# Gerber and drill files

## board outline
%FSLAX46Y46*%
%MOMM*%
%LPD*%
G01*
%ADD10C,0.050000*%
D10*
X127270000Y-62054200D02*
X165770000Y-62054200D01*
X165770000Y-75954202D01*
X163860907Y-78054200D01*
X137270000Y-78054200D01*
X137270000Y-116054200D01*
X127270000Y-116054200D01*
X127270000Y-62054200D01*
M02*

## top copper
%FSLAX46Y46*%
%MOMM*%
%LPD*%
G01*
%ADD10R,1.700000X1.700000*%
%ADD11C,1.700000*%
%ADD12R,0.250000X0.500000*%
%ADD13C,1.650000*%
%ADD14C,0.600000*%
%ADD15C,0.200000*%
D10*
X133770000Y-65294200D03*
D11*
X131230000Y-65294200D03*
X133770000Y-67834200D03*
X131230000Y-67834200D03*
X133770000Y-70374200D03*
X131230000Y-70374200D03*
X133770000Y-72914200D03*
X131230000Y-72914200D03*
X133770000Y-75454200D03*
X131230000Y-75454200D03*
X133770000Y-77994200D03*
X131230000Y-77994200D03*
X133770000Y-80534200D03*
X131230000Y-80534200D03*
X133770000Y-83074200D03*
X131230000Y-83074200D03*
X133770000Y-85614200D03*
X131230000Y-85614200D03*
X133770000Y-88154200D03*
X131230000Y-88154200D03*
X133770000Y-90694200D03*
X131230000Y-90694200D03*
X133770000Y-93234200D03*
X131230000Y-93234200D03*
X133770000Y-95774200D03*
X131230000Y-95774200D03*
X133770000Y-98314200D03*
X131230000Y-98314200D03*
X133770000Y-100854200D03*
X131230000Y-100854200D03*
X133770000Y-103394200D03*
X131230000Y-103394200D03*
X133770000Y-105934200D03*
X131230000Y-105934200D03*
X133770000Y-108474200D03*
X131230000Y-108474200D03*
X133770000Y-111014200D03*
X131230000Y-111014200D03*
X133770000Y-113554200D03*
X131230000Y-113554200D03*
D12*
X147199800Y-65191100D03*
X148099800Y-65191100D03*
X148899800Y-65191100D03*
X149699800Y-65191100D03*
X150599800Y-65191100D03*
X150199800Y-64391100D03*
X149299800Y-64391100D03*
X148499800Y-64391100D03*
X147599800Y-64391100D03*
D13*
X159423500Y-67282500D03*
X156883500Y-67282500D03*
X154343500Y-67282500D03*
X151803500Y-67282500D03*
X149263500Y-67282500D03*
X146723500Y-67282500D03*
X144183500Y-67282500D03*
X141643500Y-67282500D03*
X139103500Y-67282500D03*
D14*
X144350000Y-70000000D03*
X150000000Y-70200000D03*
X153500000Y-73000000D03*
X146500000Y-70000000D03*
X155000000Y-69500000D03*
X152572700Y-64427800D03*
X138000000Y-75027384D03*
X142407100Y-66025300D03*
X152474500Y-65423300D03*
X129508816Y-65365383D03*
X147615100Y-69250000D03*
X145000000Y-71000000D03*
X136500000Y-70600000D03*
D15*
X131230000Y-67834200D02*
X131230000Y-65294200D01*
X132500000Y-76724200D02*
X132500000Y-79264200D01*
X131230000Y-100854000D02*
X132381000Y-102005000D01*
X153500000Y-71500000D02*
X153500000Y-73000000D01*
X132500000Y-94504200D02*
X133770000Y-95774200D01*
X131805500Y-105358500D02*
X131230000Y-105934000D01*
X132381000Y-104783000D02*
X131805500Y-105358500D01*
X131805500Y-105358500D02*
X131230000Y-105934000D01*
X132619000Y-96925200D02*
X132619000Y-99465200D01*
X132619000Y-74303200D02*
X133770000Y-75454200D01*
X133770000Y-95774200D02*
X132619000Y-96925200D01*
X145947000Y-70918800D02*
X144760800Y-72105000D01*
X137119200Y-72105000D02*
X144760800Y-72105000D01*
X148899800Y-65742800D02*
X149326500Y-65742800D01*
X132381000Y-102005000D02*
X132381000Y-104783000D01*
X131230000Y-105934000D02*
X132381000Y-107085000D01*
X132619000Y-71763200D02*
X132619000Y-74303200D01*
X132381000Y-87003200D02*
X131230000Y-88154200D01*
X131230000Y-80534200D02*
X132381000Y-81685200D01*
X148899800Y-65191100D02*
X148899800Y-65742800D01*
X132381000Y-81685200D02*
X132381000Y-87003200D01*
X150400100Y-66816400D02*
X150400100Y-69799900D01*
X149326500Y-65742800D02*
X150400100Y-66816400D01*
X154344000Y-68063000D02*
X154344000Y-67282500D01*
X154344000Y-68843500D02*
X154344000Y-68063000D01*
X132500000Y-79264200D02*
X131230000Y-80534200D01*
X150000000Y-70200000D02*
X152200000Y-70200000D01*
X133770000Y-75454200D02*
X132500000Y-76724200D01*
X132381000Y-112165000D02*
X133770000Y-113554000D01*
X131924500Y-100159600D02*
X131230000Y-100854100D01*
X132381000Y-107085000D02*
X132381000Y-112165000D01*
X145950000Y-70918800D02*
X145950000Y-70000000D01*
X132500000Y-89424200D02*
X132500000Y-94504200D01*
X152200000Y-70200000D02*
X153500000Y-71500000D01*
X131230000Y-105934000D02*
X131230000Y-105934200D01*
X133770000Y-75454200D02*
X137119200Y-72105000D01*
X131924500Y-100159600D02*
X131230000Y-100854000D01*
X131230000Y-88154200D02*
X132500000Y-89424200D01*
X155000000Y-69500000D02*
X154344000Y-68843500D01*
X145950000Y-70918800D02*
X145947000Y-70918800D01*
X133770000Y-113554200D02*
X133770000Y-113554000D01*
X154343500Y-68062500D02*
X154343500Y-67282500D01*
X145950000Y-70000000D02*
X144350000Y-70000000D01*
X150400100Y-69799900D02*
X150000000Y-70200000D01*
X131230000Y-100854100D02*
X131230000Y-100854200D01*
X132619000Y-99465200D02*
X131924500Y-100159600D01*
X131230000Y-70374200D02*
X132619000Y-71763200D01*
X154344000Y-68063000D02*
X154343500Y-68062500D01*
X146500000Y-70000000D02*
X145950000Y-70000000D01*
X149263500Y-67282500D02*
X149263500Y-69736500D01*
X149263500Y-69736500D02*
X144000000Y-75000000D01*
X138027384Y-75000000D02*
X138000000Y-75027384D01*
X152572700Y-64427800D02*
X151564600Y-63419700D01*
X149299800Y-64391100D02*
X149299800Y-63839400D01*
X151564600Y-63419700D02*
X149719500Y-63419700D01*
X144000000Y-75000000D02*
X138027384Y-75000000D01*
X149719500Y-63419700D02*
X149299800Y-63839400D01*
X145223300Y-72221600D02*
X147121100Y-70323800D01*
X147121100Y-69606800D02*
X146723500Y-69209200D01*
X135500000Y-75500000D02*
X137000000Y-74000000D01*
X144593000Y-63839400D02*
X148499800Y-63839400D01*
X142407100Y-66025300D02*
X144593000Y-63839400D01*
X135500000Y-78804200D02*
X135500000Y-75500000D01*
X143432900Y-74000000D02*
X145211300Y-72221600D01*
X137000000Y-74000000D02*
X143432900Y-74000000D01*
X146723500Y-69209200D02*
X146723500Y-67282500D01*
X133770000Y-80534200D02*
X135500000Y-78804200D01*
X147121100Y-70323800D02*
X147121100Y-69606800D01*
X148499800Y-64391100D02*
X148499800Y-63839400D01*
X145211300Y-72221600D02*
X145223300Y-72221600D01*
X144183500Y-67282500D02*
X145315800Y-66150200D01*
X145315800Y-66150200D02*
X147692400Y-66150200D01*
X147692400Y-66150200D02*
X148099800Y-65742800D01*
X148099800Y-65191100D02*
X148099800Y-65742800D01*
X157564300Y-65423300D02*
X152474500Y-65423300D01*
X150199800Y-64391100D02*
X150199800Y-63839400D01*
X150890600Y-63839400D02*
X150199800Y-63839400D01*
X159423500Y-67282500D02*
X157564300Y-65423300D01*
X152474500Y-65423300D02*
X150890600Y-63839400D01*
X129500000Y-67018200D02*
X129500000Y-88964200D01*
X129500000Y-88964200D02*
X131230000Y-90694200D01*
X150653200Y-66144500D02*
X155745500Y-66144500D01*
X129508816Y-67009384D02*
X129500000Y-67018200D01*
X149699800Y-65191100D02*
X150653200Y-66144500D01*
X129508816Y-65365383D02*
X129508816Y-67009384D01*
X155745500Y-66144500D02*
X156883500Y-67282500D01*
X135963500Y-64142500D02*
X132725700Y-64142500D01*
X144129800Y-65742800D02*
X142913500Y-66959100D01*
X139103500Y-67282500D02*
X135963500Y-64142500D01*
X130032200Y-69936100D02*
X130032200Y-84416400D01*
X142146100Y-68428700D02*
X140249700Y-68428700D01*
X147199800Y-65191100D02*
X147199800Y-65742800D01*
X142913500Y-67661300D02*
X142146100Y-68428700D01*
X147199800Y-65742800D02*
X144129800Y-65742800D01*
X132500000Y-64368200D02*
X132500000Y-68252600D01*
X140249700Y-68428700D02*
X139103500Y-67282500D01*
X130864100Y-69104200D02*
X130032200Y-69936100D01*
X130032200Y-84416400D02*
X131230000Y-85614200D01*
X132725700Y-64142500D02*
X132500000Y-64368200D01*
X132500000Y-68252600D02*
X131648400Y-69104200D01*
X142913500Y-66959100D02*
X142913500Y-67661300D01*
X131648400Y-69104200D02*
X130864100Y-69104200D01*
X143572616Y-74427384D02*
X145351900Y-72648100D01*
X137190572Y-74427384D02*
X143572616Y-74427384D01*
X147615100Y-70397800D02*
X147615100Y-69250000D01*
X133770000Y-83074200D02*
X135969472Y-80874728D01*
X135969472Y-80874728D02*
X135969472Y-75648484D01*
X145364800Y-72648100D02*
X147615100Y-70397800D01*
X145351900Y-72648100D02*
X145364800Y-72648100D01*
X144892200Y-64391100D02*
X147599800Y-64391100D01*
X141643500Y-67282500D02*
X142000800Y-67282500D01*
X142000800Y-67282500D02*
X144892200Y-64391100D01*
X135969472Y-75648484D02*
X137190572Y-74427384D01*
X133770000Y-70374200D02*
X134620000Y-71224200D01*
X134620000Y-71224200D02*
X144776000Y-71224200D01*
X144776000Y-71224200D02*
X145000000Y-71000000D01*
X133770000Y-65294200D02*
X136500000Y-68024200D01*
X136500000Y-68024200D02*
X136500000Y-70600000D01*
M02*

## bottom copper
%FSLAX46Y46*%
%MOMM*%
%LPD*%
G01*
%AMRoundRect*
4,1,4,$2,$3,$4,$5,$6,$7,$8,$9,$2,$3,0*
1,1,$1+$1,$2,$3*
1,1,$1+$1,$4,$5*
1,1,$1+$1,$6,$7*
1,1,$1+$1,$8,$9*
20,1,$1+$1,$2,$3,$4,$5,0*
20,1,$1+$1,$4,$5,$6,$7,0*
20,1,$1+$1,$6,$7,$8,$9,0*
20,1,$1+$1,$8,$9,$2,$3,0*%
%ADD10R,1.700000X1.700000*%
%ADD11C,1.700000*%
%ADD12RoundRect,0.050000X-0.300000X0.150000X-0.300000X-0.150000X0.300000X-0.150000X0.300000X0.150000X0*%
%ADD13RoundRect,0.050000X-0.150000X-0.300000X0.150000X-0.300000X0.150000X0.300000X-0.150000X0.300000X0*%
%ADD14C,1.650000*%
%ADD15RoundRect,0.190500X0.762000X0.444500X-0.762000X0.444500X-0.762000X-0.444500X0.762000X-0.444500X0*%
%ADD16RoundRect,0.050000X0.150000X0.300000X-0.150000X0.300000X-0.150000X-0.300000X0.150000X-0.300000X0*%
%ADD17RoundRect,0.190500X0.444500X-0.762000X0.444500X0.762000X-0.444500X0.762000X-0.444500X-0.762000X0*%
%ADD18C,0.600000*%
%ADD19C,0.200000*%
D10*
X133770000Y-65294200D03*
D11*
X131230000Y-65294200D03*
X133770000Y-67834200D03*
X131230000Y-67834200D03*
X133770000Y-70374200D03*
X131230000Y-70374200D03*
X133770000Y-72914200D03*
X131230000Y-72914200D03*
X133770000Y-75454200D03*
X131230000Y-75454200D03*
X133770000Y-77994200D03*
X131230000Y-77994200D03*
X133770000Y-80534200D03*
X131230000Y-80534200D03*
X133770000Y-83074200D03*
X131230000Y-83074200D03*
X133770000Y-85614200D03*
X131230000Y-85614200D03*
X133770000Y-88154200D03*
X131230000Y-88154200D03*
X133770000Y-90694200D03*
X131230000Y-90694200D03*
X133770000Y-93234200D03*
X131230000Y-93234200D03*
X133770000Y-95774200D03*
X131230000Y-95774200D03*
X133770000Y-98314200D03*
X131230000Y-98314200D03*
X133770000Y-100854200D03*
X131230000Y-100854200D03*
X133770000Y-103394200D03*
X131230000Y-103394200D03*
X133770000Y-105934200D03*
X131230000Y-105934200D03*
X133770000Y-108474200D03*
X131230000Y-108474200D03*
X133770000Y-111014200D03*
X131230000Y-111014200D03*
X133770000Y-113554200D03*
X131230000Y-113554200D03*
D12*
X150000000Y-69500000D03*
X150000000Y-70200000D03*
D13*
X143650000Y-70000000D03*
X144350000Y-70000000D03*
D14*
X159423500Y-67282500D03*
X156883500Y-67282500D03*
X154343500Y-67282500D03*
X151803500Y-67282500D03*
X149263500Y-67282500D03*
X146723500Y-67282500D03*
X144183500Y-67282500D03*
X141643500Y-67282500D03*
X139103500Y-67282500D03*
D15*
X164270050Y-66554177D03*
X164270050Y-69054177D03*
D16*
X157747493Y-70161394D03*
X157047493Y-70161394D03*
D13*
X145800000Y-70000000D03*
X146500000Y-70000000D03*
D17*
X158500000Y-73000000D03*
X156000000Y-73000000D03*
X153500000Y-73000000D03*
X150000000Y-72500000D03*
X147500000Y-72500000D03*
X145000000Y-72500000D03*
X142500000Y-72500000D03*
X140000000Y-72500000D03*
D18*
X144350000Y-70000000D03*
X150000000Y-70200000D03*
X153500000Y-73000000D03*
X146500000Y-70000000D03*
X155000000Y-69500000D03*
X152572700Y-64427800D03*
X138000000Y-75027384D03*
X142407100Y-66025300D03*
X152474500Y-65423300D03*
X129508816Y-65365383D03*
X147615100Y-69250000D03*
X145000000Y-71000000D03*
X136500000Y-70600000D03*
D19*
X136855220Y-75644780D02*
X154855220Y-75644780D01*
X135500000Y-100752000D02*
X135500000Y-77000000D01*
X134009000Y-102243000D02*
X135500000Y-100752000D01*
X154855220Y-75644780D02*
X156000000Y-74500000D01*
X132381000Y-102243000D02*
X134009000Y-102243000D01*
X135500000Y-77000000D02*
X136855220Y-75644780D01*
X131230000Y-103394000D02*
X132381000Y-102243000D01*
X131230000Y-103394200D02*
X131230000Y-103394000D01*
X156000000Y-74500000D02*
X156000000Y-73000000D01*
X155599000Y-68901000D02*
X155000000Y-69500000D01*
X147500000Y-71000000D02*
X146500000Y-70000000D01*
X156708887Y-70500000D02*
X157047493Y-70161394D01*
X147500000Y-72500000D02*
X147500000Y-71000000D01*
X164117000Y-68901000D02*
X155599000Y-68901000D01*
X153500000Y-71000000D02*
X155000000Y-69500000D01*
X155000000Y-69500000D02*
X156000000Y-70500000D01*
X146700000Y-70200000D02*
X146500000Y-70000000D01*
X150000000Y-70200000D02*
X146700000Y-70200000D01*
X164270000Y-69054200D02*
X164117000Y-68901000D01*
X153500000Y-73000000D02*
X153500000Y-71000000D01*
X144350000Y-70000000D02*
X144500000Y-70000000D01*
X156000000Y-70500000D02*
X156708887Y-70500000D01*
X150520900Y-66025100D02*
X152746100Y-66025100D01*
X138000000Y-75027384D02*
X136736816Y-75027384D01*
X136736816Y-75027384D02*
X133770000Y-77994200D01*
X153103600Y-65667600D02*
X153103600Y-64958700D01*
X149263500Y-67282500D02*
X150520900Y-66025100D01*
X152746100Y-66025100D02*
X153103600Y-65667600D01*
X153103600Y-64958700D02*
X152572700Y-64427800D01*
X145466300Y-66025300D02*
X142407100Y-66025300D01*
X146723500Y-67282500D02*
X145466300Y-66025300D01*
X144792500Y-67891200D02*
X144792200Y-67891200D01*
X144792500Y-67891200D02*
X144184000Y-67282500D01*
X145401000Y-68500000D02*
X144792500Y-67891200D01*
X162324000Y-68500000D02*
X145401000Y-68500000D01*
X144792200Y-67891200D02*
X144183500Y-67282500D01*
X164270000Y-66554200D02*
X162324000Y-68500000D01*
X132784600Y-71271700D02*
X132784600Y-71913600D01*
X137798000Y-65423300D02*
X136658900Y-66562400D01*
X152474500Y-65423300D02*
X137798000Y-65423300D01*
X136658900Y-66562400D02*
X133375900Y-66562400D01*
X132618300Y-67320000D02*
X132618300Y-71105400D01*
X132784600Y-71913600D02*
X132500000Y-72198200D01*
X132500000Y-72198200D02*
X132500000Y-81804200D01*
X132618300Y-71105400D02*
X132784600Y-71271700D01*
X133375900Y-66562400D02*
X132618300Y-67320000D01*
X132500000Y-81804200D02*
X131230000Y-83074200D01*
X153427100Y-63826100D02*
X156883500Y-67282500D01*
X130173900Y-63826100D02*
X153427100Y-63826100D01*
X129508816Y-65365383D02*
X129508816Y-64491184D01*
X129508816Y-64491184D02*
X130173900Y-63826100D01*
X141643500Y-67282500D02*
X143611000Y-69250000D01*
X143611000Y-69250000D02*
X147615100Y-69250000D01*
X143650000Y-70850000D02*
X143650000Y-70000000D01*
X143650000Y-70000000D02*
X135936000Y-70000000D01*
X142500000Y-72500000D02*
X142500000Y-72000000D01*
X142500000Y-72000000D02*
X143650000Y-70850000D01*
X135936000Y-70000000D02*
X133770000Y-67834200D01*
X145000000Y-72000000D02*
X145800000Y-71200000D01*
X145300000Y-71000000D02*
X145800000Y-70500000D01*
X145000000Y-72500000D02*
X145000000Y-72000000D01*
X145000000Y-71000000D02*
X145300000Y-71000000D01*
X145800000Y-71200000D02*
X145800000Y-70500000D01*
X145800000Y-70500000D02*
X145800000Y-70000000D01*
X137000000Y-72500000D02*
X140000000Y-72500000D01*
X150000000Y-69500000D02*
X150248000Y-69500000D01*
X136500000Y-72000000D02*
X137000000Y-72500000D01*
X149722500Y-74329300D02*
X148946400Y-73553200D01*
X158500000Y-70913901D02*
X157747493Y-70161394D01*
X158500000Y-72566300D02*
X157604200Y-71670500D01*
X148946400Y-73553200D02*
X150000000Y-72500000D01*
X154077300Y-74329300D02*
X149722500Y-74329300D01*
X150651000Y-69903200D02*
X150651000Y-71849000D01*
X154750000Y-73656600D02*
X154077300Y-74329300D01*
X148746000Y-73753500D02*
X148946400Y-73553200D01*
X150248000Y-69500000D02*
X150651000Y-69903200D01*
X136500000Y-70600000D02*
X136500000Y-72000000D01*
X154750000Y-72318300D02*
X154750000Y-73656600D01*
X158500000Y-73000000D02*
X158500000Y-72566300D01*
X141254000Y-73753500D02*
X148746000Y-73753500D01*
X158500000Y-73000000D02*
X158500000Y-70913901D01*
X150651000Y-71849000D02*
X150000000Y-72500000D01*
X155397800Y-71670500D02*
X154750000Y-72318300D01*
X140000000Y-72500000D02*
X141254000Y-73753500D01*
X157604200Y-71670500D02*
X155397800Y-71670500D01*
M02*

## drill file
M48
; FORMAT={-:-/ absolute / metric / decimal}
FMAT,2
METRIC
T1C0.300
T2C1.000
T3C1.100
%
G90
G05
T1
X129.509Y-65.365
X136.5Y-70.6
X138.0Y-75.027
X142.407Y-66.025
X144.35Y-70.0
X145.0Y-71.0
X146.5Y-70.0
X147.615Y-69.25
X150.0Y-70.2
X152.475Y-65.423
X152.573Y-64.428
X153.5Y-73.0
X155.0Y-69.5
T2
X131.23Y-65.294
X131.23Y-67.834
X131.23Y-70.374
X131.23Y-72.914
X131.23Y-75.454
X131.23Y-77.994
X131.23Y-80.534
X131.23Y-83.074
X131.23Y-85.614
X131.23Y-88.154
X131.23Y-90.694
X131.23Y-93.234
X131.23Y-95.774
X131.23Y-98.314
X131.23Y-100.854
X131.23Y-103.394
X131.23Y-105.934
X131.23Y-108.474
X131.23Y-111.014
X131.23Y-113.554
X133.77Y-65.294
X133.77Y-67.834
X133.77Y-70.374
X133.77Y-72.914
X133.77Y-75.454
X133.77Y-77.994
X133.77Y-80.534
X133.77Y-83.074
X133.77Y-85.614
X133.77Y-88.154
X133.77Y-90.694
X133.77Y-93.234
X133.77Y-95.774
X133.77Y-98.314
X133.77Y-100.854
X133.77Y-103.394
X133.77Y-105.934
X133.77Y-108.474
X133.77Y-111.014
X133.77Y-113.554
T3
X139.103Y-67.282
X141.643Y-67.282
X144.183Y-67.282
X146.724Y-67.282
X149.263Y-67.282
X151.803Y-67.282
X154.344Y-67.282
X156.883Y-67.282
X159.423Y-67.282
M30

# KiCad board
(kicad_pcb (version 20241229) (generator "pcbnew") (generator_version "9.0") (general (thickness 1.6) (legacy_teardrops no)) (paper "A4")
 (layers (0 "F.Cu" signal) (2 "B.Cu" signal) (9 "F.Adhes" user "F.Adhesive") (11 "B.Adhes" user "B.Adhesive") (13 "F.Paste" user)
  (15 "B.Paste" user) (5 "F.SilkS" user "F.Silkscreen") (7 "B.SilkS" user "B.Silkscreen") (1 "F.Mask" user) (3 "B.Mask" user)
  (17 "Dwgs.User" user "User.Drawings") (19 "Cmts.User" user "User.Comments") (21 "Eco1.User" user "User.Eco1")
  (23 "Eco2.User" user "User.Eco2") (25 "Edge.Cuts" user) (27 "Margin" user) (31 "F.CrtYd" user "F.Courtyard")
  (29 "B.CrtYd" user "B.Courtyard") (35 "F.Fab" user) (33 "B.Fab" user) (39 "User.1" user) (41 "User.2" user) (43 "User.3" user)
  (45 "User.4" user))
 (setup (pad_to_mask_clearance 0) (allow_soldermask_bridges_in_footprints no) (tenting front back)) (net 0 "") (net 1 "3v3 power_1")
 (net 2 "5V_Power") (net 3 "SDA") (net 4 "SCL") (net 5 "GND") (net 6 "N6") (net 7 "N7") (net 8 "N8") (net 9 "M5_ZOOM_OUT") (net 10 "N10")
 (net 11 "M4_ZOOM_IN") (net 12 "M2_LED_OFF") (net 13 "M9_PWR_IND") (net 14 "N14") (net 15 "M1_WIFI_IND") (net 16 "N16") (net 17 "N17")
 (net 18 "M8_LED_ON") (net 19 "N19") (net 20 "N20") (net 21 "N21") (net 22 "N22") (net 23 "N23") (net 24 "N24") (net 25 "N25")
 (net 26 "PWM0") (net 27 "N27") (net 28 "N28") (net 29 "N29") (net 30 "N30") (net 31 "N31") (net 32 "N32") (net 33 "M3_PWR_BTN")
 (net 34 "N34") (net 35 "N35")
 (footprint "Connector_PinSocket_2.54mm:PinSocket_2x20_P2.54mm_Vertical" (layer "F.Cu") (at 133.77 65.2942)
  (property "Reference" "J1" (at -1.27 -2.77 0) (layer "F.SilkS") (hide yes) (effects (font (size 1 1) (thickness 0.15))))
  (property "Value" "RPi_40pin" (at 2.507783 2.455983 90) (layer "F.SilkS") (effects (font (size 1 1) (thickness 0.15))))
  (pad "1" thru_hole rect (at 0 0) (size 1.7 1.7) (drill 1) (layers "*.Cu" "*.Mask") (remove_unused_layers no) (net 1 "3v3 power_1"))
  (pad "2" thru_hole circle (at -2.54 0) (size 1.7 1.7) (drill 1) (layers "*.Cu" "*.Mask") (remove_unused_layers no) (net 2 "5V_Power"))
  (pad "3" thru_hole circle (at 0 2.54) (size 1.7 1.7) (drill 1) (layers "*.Cu" "*.Mask") (remove_unused_layers no) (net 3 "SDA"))
  (pad "4" thru_hole circle (at -2.54 2.54) (size 1.7 1.7) (drill 1) (layers "*.Cu" "*.Mask") (remove_unused_layers no) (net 2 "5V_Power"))
  (pad "5" thru_hole circle (at 0 5.08) (size 1.7 1.7) (drill 1) (layers "*.Cu" "*.Mask") (remove_unused_layers no) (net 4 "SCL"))
  (pad "6" thru_hole circle (at -2.54 5.08) (size 1.7 1.7) (drill 1) (layers "*.Cu" "*.Mask") (remove_unused_layers no) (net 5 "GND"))
  (pad "7" thru_hole circle (at 0 7.62) (size 1.7 1.7) (drill 1) (layers "*.Cu" "*.Mask") (remove_unused_layers no) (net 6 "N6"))
  (pad "8" thru_hole circle (at -2.54 7.62) (size 1.7 1.7) (drill 1) (layers "*.Cu" "*.Mask") (remove_unused_layers no) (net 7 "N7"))
  (pad "9" thru_hole circle (at 0 10.16) (size 1.7 1.7) (drill 1) (layers "*.Cu" "*.Mask") (remove_unused_layers no) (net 5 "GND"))
  (pad "10" thru_hole circle (at -2.54 10.16) (size 1.7 1.7) (drill 1) (layers "*.Cu" "*.Mask") (remove_unused_layers no) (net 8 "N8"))
  (pad "11" thru_hole circle (at 0 12.7) (size 1.7 1.7) (drill 1) (layers "*.Cu" "*.Mask") (remove_unused_layers no) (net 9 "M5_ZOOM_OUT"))
  (pad "12" thru_hole circle (at -2.54 12.7) (size 1.7 1.7) (drill 1) (layers "*.Cu" "*.Mask") (remove_unused_layers no) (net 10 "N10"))
  (pad "13" thru_hole circle (at 0 15.24) (size 1.7 1.7) (drill 1) (layers "*.Cu" "*.Mask") (remove_unused_layers no) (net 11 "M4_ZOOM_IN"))
  (pad "14" thru_hole circle (at -2.54 15.24) (size 1.7 1.7) (drill 1) (layers "*.Cu" "*.Mask") (remove_unused_layers no) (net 5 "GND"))
  (pad "15" thru_hole circle (at 0 17.78) (size 1.7 1.7) (drill 1) (layers "*.Cu" "*.Mask") (remove_unused_layers no) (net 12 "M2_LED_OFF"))
  (pad "16" thru_hole circle (at -2.54 17.78) (size 1.7 1.7) (drill 1) (layers "*.Cu" "*.Mask") (remove_unused_layers no)
   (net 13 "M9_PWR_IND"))
  (pad "17" thru_hole circle (at 0 20.32) (size 1.7 1.7) (drill 1) (layers "*.Cu" "*.Mask") (remove_unused_layers no) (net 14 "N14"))
  (pad "18" thru_hole circle (at -2.54 20.32) (size 1.7 1.7) (drill 1) (layers "*.Cu" "*.Mask") (remove_unused_layers no)
   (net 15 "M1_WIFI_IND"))
  (pad "19" thru_hole circle (at 0 22.86) (size 1.7 1.7) (drill 1) (layers "*.Cu" "*.Mask") (remove_unused_layers no) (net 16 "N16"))
  (pad "20" thru_hole circle (at -2.54 22.86) (size 1.7 1.7) (drill 1) (layers "*.Cu" "*.Mask") (remove_unused_layers no) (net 5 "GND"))
  (pad "21" thru_hole circle (at 0 25.4) (size 1.7 1.7) (drill 1) (layers "*.Cu" "*.Mask") (remove_unused_layers no) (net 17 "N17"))
  (pad "22" thru_hole circle (at -2.54 25.4) (size 1.7 1.7) (drill 1) (layers "*.Cu" "*.Mask") (remove_unused_layers no)
   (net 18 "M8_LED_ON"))
  (pad "23" thru_hole circle (at 0 27.94) (size 1.7 1.7) (drill 1) (layers "*.Cu" "*.Mask") (remove_unused_layers no) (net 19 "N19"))
  (pad "24" thru_hole circle (at -2.54 27.94) (size 1.7 1.7) (drill 1) (layers "*.Cu" "*.Mask") (remove_unused_layers no) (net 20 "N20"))
  (pad "25" thru_hole circle (at 0 30.48) (size 1.7 1.7) (drill 1) (layers "*.Cu" "*.Mask") (remove_unused_layers no) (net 5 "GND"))
  (pad "26" thru_hole circle (at -2.54 30.48) (size 1.7 1.7) (drill 1) (layers "*.Cu" "*.Mask") (remove_unused_layers no) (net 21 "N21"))
  (pad "27" thru_hole circle (at 0 33.02) (size 1.7 1.7) (drill 1) (layers "*.Cu" "*.Mask") (remove_unused_layers no) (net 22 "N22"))
  (pad "28" thru_hole circle (at -2.54 33.02) (size 1.7 1.7) (drill 1) (layers "*.Cu" "*.Mask") (remove_unused_layers no) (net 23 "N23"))
  (pad "29" thru_hole circle (at 0 35.56) (size 1.7 1.7) (drill 1) (layers "*.Cu" "*.Mask") (remove_unused_layers no) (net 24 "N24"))
  (pad "30" thru_hole circle (at -2.54 35.56) (size 1.7 1.7) (drill 1) (layers "*.Cu" "*.Mask") (remove_unused_layers no) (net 5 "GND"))
  (pad "31" thru_hole circle (at 0 38.1) (size 1.7 1.7) (drill 1) (layers "*.Cu" "*.Mask") (remove_unused_layers no) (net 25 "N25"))
  (pad "32" thru_hole circle (at -2.54 38.1) (size 1.7 1.7) (drill 1) (layers "*.Cu" "*.Mask") (remove_unused_layers no) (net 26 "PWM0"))
  (pad "33" thru_hole circle (at 0 40.64) (size 1.7 1.7) (drill 1) (layers "*.Cu" "*.Mask") (remove_unused_layers no) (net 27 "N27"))
  (pad "34" thru_hole circle (at -2.54 40.64) (size 1.7 1.7) (drill 1) (layers "*.Cu" "*.Mask") (remove_unused_layers no) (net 5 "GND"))
  (pad "35" thru_hole circle (at 0 43.18) (size 1.7 1.7) (drill 1) (layers "*.Cu" "*.Mask") (remove_unused_layers no) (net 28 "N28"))
  (pad "36" thru_hole circle (at -2.54 43.18) (size 1.7 1.7) (drill 1) (layers "*.Cu" "*.Mask") (remove_unused_layers no) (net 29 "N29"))
  (pad "37" thru_hole circle (at 0 45.72) (size 1.7 1.7) (drill 1) (layers "*.Cu" "*.Mask") (remove_unused_layers no) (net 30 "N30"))
  (pad "38" thru_hole circle (at -2.54 45.72) (size 1.7 1.7) (drill 1) (layers "*.Cu" "*.Mask") (remove_unused_layers no) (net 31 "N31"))
  (pad "39" thru_hole circle (at 0 48.26) (size 1.7 1.7) (drill 1) (layers "*.Cu" "*.Mask") (remove_unused_layers no) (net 5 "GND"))
  (pad "40" thru_hole circle (at -2.54 48.26) (size 1.7 1.7) (drill 1) (layers "*.Cu" "*.Mask") (remove_unused_layers no) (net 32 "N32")))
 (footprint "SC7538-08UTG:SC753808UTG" (layer "F.Cu") (at 148.8998 64.7911)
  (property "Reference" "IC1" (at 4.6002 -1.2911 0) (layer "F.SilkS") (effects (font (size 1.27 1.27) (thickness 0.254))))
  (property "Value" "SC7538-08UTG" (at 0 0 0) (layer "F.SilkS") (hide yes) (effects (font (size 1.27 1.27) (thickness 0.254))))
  (pad "1" smd rect (at -1.7 0.4) (size 0.25 0.5) (layers "F.Cu" "F.Mask" "F.Paste") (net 15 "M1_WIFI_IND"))
  (pad "2" smd rect (at -0.8 0.4) (size 0.25 0.5) (layers "F.Cu" "F.Mask" "F.Paste") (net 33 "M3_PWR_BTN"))
  (pad "3" smd rect (at 0 0.4) (size 0.25 0.5) (layers "F.Cu" "F.Mask" "F.Paste") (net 5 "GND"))
  (pad "4" smd rect (at 0.8 0.4) (size 0.25 0.5) (layers "F.Cu" "F.Mask" "F.Paste") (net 18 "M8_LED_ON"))
  (pad "5" smd rect (at 1.7 0.4) (size 0.25 0.5) (layers "F.Cu" "F.Mask" "F.Paste") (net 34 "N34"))
  (pad "6" smd rect (at 1.3 -0.4) (size 0.25 0.5) (layers "F.Cu" "F.Mask" "F.Paste") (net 13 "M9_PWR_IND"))
  (pad "7" smd rect (at 0.4 -0.4) (size 0.25 0.5) (layers "F.Cu" "F.Mask" "F.Paste") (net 9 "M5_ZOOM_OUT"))
  (pad "8" smd rect (at -0.4 -0.4) (size 0.25 0.5) (layers "F.Cu" "F.Mask" "F.Paste") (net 11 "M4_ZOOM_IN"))
  (pad "9" smd rect (at -1.3 -0.4) (size 0.25 0.5) (layers "F.Cu" "F.Mask" "F.Paste") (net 12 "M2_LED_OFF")))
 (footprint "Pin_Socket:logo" (layer "B.Cu") (at 159.5 76.5 180)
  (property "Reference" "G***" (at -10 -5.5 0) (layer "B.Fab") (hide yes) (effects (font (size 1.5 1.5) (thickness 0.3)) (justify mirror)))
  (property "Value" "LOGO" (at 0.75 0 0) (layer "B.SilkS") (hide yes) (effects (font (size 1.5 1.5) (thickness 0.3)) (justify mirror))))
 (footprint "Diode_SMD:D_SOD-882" (layer "B.Cu") (at 150 69.85 -90)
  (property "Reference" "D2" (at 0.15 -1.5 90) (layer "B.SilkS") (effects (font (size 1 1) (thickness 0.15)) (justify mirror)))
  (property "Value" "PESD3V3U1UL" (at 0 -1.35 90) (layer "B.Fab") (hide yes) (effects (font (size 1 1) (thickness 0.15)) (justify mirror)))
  (pad "" smd roundrect (at -0.35 0 270) (size 0.3 0.6) (layers "B.Paste") (roundrect_rratio 0.1666666667) (solder_paste_margin -0.05))
  (pad "" smd roundrect (at 0.35 0 270) (size 0.3 0.6) (layers "B.Paste") (roundrect_rratio 0.1666666667) (solder_paste_margin -0.05))
  (pad "1" smd roundrect (at -0.35 0 270) (size 0.4 0.7) (layers "B.Cu" "B.Mask") (roundrect_rratio 0.125) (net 1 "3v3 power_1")
   (solder_paste_margin -0.05))
  (pad "2" smd roundrect (at 0.35 0 270) (size 0.4 0.7) (layers "B.Cu" "B.Mask") (roundrect_rratio 0.125) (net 5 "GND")
   (solder_paste_margin -0.05)))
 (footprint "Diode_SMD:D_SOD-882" (layer "B.Cu") (at 144 70)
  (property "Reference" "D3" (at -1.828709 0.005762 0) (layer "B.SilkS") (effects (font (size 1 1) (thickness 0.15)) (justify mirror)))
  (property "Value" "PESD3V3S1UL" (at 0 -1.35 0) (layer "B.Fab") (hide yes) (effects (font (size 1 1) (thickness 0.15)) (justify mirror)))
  (pad "" smd roundrect (at -0.35 0) (size 0.3 0.6) (layers "B.Paste") (roundrect_rratio 0.1666666667) (solder_paste_margin -0.05))
  (pad "" smd roundrect (at 0.35 0) (size 0.3 0.6) (layers "B.Paste") (roundrect_rratio 0.1666666667) (solder_paste_margin -0.05))
  (pad "1" smd roundrect (at -0.35 0) (size 0.4 0.7) (layers "B.Cu" "B.Mask") (roundrect_rratio 0.125) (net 3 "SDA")
   (solder_paste_margin -0.05))
  (pad "2" smd roundrect (at 0.35 0) (size 0.4 0.7) (layers "B.Cu" "B.Mask") (roundrect_rratio 0.125) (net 5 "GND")
   (solder_paste_margin -0.05)))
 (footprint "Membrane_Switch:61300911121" (layer "B.Cu") (at 149.2635 67.2825 180)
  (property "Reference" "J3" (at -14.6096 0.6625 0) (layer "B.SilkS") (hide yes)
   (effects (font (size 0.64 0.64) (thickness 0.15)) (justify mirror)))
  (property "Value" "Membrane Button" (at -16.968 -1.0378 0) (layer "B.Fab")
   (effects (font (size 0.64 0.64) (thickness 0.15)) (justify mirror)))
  (pad "1" thru_hole circle (at -10.16 0 180) (size 1.65 1.65) (drill 1.1) (layers "*.Cu" "*.Mask") (remove_unused_layers no)
   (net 13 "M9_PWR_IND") (solder_mask_margin 0.102))
  (pad "2" thru_hole circle (at -7.62 0 180) (size 1.65 1.65) (drill 1.1) (layers "*.Cu" "*.Mask") (remove_unused_layers no)
   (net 18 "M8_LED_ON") (solder_mask_margin 0.102))
  (pad "3" thru_hole circle (at -5.08 0 180) (size 1.65 1.65) (drill 1.1) (layers "*.Cu" "*.Mask") (remove_unused_layers no) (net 5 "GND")
   (solder_mask_margin 0.102))
  (pad "4" thru_hole circle (at -2.54 0 180) (size 1.65 1.65) (drill 1.1) (layers "*.Cu" "*.Mask") (remove_unused_layers no) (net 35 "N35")
   (solder_mask_margin 0.102))
  (pad "5" thru_hole circle (at 0 0 180) (size 1.65 1.65) (drill 1.1) (layers "*.Cu" "*.Mask") (remove_unused_layers no)
   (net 9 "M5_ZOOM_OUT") (solder_mask_margin 0.102))
  (pad "6" thru_hole circle (at 2.54 0 180) (size 1.65 1.65) (drill 1.1) (layers "*.Cu" "*.Mask") (remove_unused_layers no)
   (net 11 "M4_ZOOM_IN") (solder_mask_margin 0.102))
  (pad "7" thru_hole circle (at 5.08 0 180) (size 1.65 1.65) (drill 1.1) (layers "*.Cu" "*.Mask") (remove_unused_layers no)
   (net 33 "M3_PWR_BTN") (solder_mask_margin 0.102))
  (pad "8" thru_hole circle (at 7.62 0 180) (size 1.65 1.65) (drill 1.1) (layers "*.Cu" "*.Mask") (remove_unused_layers no)
   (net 12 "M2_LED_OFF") (solder_mask_margin 0.102))
  (pad "9" thru_hole circle (at 10.16 0 180) (size 1.65 1.65) (drill 1.1) (layers "*.Cu" "*.Mask") (remove_unused_layers no)
   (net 15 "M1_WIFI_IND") (solder_mask_margin 0.102)))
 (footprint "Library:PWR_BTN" (layer "B.Cu") (at 163.7823 67.8148 -90)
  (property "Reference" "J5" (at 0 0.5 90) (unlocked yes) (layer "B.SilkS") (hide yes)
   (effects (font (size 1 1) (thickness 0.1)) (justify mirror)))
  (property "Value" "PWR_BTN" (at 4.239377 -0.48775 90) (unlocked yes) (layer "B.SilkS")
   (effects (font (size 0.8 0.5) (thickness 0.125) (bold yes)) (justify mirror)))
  (pad "1" smd roundrect (at -1.260623 -0.48775 180) (size 1.905 1.27) (layers "B.Cu" "B.Mask" "B.Paste") (roundrect_rratio 0.15)
   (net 33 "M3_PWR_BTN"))
  (pad "2" smd roundrect (at 1.239377 -0.48775 180) (size 1.905 1.27) (layers "B.Cu" "B.Mask" "B.Paste") (roundrect_rratio 0.15)
   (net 5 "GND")))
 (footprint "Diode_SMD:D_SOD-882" (layer "B.Cu") (at 157.397493 70.161394 180)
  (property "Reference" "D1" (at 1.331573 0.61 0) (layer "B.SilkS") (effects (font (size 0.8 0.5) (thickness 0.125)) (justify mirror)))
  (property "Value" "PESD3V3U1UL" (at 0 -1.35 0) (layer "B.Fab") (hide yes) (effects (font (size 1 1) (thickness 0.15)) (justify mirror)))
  (pad "" smd roundrect (at -0.35 0 180) (size 0.3 0.6) (layers "B.Paste") (roundrect_rratio 0.1666666667) (solder_paste_margin -0.05))
  (pad "" smd roundrect (at 0.35 0 180) (size 0.3 0.6) (layers "B.Paste") (roundrect_rratio 0.1666666667) (solder_paste_margin -0.05))
  (pad "1" smd roundrect (at -0.35 0 180) (size 0.4 0.7) (layers "B.Cu" "B.Mask") (roundrect_rratio 0.125) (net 1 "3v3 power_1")
   (solder_paste_margin -0.05))
  (pad "2" smd roundrect (at 0.35 0 180) (size 0.4 0.7) (layers "B.Cu" "B.Mask") (roundrect_rratio 0.125) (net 5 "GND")
   (solder_paste_margin -0.05)))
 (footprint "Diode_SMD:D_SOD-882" (layer "B.Cu") (at 146.15 70)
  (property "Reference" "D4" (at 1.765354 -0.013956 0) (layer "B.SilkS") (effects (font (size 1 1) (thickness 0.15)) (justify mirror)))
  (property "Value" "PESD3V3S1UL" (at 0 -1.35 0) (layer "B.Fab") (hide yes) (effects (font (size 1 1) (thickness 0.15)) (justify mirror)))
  (pad "" smd roundrect (at -0.35 0) (size 0.3 0.6) (layers "B.Paste") (roundrect_rratio 0.1666666667) (solder_paste_margin -0.05))
  (pad "" smd roundrect (at 0.35 0) (size 0.3 0.6) (layers "B.Paste") (roundrect_rratio 0.1666666667) (solder_paste_margin -0.05))
  (pad "1" smd roundrect (at -0.35 0) (size 0.4 0.7) (layers "B.Cu" "B.Mask") (roundrect_rratio 0.125) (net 4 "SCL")
   (solder_paste_margin -0.05))
  (pad "2" smd roundrect (at 0.35 0) (size 0.4 0.7) (layers "B.Cu" "B.Mask") (roundrect_rratio 0.125) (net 5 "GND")
   (solder_paste_margin -0.05)))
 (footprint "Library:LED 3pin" (layer "B.Cu") (at 156 73 180)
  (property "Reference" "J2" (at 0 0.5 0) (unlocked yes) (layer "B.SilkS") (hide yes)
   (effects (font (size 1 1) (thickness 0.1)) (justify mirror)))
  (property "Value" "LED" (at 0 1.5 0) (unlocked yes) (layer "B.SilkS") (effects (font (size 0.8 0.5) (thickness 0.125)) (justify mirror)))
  (pad "1" smd roundrect (at -2.5 0 90) (size 1.905 1.27) (layers "B.Cu" "B.Mask" "B.Paste") (roundrect_rratio 0.15) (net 1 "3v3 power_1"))
  (pad "2" smd roundrect (at 0 0 90) (size 1.905 1.27) (layers "B.Cu" "B.Mask" "B.Paste") (roundrect_rratio 0.15) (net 26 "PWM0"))
  (pad "3" smd roundrect (at 2.5 0 90) (size 1.905 1.27) (layers "B.Cu" "B.Mask" "B.Paste") (roundrect_rratio 0.15) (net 5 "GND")))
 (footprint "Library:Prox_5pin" (layer "B.Cu") (at 145 72.5 180)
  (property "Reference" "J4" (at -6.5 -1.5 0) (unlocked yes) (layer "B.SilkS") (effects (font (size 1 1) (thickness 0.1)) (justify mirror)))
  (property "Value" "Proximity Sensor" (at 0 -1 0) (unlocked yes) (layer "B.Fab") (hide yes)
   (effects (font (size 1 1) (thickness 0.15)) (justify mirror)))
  (pad "1" smd roundrect (at -5 0 90) (size 1.905 1.27) (layers "B.Cu" "B.Mask" "B.Paste") (roundrect_rratio 0.15) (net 1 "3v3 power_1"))
  (pad "2" smd roundrect (at -2.5 0 90) (size 1.905 1.27) (layers "B.Cu" "B.Mask" "B.Paste") (roundrect_rratio 0.15) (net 5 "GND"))
  (pad "3" smd roundrect (at 0 0 90) (size 1.905 1.27) (layers "B.Cu" "B.Mask" "B.Paste") (roundrect_rratio 0.15) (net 4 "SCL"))
  (pad "4" smd roundrect (at 2.5 0 90) (size 1.905 1.27) (layers "B.Cu" "B.Mask" "B.Paste") (roundrect_rratio 0.15) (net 3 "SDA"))
  (pad "5" smd roundrect (at 5 0 90) (size 1.905 1.27) (layers "B.Cu" "B.Mask" "B.Paste") (roundrect_rratio 0.15) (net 1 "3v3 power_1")))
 (gr_poly
  (pts (xy 127.27 62.0542) (xy 165.77 62.0542) (xy 165.77 75.954202) (xy 163.860907 78.0542) (xy 137.27 78.0542) (xy 137.27 116.0542)
   (xy 127.27 116.0542))
  (stroke (width 0.05) (type solid)) (fill no) (layer "Edge.Cuts"))
 (segment (start 131.23 67.8342) (end 131.23 65.2942) (width 0.2) (layer "F.Cu") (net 2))
 (segment (start 136.85522 75.64478) (end 154.85522 75.64478) (width 0.2) (layer "B.Cu") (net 26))
 (segment (start 135.5 100.752) (end 135.5 77) (width 0.2) (layer "B.Cu") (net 26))
 (segment (start 134.009 102.243) (end 135.5 100.752) (width 0.2) (layer "B.Cu") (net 26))
 (segment (start 154.85522 75.64478) (end 156 74.5) (width 0.2) (layer "B.Cu") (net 26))
 (segment (start 132.381 102.243) (end 134.009 102.243) (width 0.2) (layer "B.Cu") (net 26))
 (segment (start 135.5 77) (end 136.85522 75.64478) (width 0.2) (layer "B.Cu") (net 26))
 (segment (start 131.23 103.394) (end 132.381 102.243) (width 0.2) (layer "B.Cu") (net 26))
 (segment (start 131.23 103.3942) (end 131.23 103.394) (width 0.2) (layer "B.Cu") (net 26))
 (segment (start 156 74.5) (end 156 73) (width 0.2) (layer "B.Cu") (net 26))
 (segment (start 132.5 76.7242) (end 132.5 79.2642) (width 0.2) (layer "F.Cu") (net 5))
 (segment (start 131.23 100.854) (end 132.381 102.005) (width 0.2) (layer "F.Cu") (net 5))
 (segment (start 153.5 71.5) (end 153.5 73) (width 0.2) (layer "F.Cu") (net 5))
 (segment (start 132.5 94.5042) (end 133.77 95.7742) (width 0.2) (layer "F.Cu") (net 5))
 (segment (start 131.8055 105.3585) (end 131.23 105.934) (width 0.2) (layer "F.Cu") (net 5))
 (segment (start 132.381 104.783) (end 131.8055 105.3585) (width 0.2) (layer "F.Cu") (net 5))
 (segment (start 131.8055 105.3585) (end 131.23 105.934) (width 0.2) (layer "F.Cu") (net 5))
 (segment (start 132.619 96.9252) (end 132.619 99.4652) (width 0.2) (layer "F.Cu") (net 5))
 (segment (start 132.619 74.3032) (end 133.77 75.4542) (width 0.2) (layer "F.Cu") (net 5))
 (segment (start 133.77 95.7742) (end 132.619 96.9252) (width 0.2) (layer "F.Cu") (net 5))
 (segment (start 145.947 70.9188) (end 144.7608 72.105) (width 0.2) (layer "F.Cu") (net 5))
 (segment (start 137.1192 72.105) (end 144.7608 72.105) (width 0.2) (layer "F.Cu") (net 5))
 (segment (start 148.8998 65.7428) (end 149.3265 65.7428) (width 0.2) (layer "F.Cu") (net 5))
 (segment (start 132.381 102.005) (end 132.381 104.783) (width 0.2) (layer "F.Cu") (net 5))
 (segment (start 131.23 105.934) (end 132.381 107.085) (width 0.2) (layer "F.Cu") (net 5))
 (segment (start 132.619 71.7632) (end 132.619 74.3032) (width 0.2) (layer "F.Cu") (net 5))
 (segment (start 132.381 87.0032) (end 131.23 88.1542) (width 0.2) (layer "F.Cu") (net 5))
 (segment (start 131.23 80.5342) (end 132.381 81.6852) (width 0.2) (layer "F.Cu") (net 5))
 (segment (start 148.8998 65.1911) (end 148.8998 65.7428) (width 0.2) (layer "F.Cu") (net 5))
 (segment (start 132.381 81.6852) (end 132.381 87.0032) (width 0.2) (layer "F.Cu") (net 5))
 (segment (start 150.4001 66.8164) (end 150.4001 69.7999) (width 0.2) (layer "F.Cu") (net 5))
 (segment (start 149.3265 65.7428) (end 150.4001 66.8164) (width 0.2) (layer "F.Cu") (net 5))
 (segment (start 154.344 68.063) (end 154.344 67.2825) (width 0.2) (layer "F.Cu") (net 5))
 (segment (start 154.344 68.8435) (end 154.344 68.063) (width 0.2) (layer "F.Cu") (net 5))
 (segment (start 132.5 79.2642) (end 131.23 80.5342) (width 0.2) (layer "F.Cu") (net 5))
 (segment (start 150 70.2) (end 152.2 70.2) (width 0.2) (layer "F.Cu") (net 5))
 (segment (start 133.77 75.4542) (end 132.5 76.7242) (width 0.2) (layer "F.Cu") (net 5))
 (segment (start 132.381 112.165) (end 133.77 113.554) (width 0.2) (layer "F.Cu") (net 5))
 (segment (start 131.9245 100.1596) (end 131.23 100.8541) (width 0.2) (layer "F.Cu") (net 5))
 (segment (start 132.381 107.085) (end 132.381 112.165) (width 0.2) (layer "F.Cu") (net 5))
 (segment (start 145.95 70.9188) (end 145.95 70) (width 0.2) (layer "F.Cu") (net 5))
 (segment (start 132.5 89.4242) (end 132.5 94.5042) (width 0.2) (layer "F.Cu") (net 5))
 (segment (start 152.2 70.2) (end 153.5 71.5) (width 0.2) (layer "F.Cu") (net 5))
 (segment (start 131.23 105.934) (end 131.23 105.9342) (width 0.2) (layer "F.Cu") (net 5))
 (segment (start 133.77 75.4542) (end 137.1192 72.105) (width 0.2) (layer "F.Cu") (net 5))
 (segment (start 131.9245 100.1596) (end 131.23 100.854) (width 0.2) (layer "F.Cu") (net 5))
 (segment (start 131.23 88.1542) (end 132.5 89.4242) (width 0.2) (layer "F.Cu") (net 5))
 (segment (start 155 69.5) (end 154.344 68.8435) (width 0.2) (layer "F.Cu") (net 5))
 (segment (start 145.95 70.9188) (end 145.947 70.9188) (width 0.2) (layer "F.Cu") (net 5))
 (segment (start 133.77 113.5542) (end 133.77 113.554) (width 0.2) (layer "F.Cu") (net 5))
 (segment (start 154.3435 68.0625) (end 154.3435 67.2825) (width 0.2) (layer "F.Cu") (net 5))
 (segment (start 145.95 70) (end 144.35 70) (width 0.2) (layer "F.Cu") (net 5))
 (segment (start 150.4001 69.7999) (end 150 70.2) (width 0.2) (layer "F.Cu") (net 5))
 (segment (start 131.23 100.8541) (end 131.23 100.8542) (width 0.2) (layer "F.Cu") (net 5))
 (segment (start 132.619 99.4652) (end 131.9245 100.1596) (width 0.2) (layer "F.Cu") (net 5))
 (segment (start 131.23 70.3742) (end 132.619 71.7632) (width 0.2) (layer "F.Cu") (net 5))
 (segment (start 154.344 68.063) (end 154.3435 68.0625) (width 0.2) (layer "F.Cu") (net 5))
 (segment (start 146.5 70) (end 145.95 70) (width 0.2) (layer "F.Cu") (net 5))
 (via (at 144.35 70) (size 0.6) (drill 0.3) (layers "F.Cu" "B.Cu") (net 5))
 (via (at 150 70.2) (size 0.6) (drill 0.3) (layers "F.Cu" "B.Cu") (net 5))
 (via (at 153.5 73) (size 0.6) (drill 0.3) (layers "F.Cu" "B.Cu") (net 5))
 (via (at 146.5 70) (size 0.6) (drill 0.3) (layers "F.Cu" "B.Cu") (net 5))
 (via (at 155 69.5) (size 0.6) (drill 0.3) (layers "F.Cu" "B.Cu") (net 5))
 (segment (start 155.599 68.901) (end 155 69.5) (width 0.2) (layer "B.Cu") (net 5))
 (segment (start 147.5 71) (end 146.5 70) (width 0.2) (layer "B.Cu") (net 5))
 (segment (start 156.708887 70.5) (end 157.047493 70.161394) (width 0.2) (layer "B.Cu") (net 5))
 (segment (start 147.5 72.5) (end 147.5 71) (width 0.2) (layer "B.Cu") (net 5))
 (segment (start 164.117 68.901) (end 155.599 68.901) (width 0.2) (layer "B.Cu") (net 5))
 (segment (start 153.5 71) (end 155 69.5) (width 0.2) (layer "B.Cu") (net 5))
 (segment (start 155 69.5) (end 156 70.5) (width 0.2) (layer "B.Cu") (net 5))
 (segment (start 146.7 70.2) (end 146.5 70) (width 0.2) (layer "B.Cu") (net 5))
 (segment (start 150 70.2) (end 146.7 70.2) (width 0.2) (layer "B.Cu") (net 5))
 (segment (start 164.27 69.0542) (end 164.117 68.901) (width 0.2) (layer "B.Cu") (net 5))
 (segment (start 153.5 73) (end 153.5 71) (width 0.2) (layer "B.Cu") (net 5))
 (segment (start 144.35 70) (end 144.5 70) (width 0.2) (layer "B.Cu") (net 5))
 (segment (start 156 70.5) (end 156.708887 70.5) (width 0.2) (layer "B.Cu") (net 5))
 (segment (start 149.2635 67.2825) (end 149.2635 69.7365) (width 0.2) (layer "F.Cu") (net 9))
 (segment (start 149.2635 69.7365) (end 144 75) (width 0.2) (layer "F.Cu") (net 9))
 (segment (start 138.027384 75) (end 138 75.027384) (width 0.2) (layer "F.Cu") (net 9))
 (segment (start 152.5727 64.4278) (end 151.5646 63.4197) (width 0.2) (layer "F.Cu") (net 9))
 (segment (start 149.2998 64.3911) (end 149.2998 63.8394) (width 0.2) (layer "F.Cu") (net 9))
 (segment (start 151.5646 63.4197) (end 149.7195 63.4197) (width 0.2) (layer "F.Cu") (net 9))
 (segment (start 144 75) (end 138.027384 75) (width 0.2) (layer "F.Cu") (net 9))
 (segment (start 149.7195 63.4197) (end 149.2998 63.8394) (width 0.2) (layer "F.Cu") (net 9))
 (via (at 152.5727 64.4278) (size 0.6) (drill 0.3) (layers "F.Cu" "B.Cu") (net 9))
 (via (at 138 75.027384) (size 0.6) (drill 0.3) (layers "F.Cu" "B.Cu") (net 9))
 (segment (start 150.5209 66.0251) (end 152.7461 66.0251) (width 0.2) (layer "B.Cu") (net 9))
 (segment (start 138 75.027384) (end 136.736816 75.027384) (width 0.2) (layer "B.Cu") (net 9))
 (segment (start 136.736816 75.027384) (end 133.77 77.9942) (width 0.2) (layer "B.Cu") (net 9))
 (segment (start 153.1036 65.6676) (end 153.1036 64.9587) (width 0.2) (layer "B.Cu") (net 9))
 (segment (start 149.2635 67.2825) (end 150.5209 66.0251) (width 0.2) (layer "B.Cu") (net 9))
 (segment (start 152.7461 66.0251) (end 153.1036 65.6676) (width 0.2) (layer "B.Cu") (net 9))
 (segment (start 153.1036 64.9587) (end 152.5727 64.4278) (width 0.2) (layer "B.Cu") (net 9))
 (segment (start 145.2233 72.2216) (end 147.1211 70.3238) (width 0.2) (layer "F.Cu") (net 11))
 (segment (start 147.1211 69.6068) (end 146.7235 69.2092) (width 0.2) (layer "F.Cu") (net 11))
 (segment (start 135.5 75.5) (end 137 74) (width 0.2) (layer "F.Cu") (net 11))
 (segment (start 144.593 63.8394) (end 148.4998 63.8394) (width 0.2) (layer "F.Cu") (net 11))
 (segment (start 142.4071 66.0253) (end 144.593 63.8394) (width 0.2) (layer "F.Cu") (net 11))
 (segment (start 135.5 78.8042) (end 135.5 75.5) (width 0.2) (layer "F.Cu") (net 11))
 (segment (start 143.4329 74) (end 145.2113 72.2216) (width 0.2) (layer "F.Cu") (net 11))
 (segment (start 137 74) (end 143.4329 74) (width 0.2) (layer "F.Cu") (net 11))
 (segment (start 146.7235 69.2092) (end 146.7235 67.2825) (width 0.2) (layer "F.Cu") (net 11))
 (segment (start 133.77 80.5342) (end 135.5 78.8042) (width 0.2) (layer "F.Cu") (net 11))
 (segment (start 147.1211 70.3238) (end 147.1211 69.6068) (width 0.2) (layer "F.Cu") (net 11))
 (segment (start 148.4998 64.3911) (end 148.4998 63.8394) (width 0.2) (layer "F.Cu") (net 11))
 (segment (start 145.2113 72.2216) (end 145.2233 72.2216) (width 0.2) (layer "F.Cu") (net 11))
 (via (at 142.4071 66.0253) (size 0.6) (drill 0.3) (layers "F.Cu" "B.Cu") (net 11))
 (segment (start 145.4663 66.0253) (end 142.4071 66.0253) (width 0.2) (layer "B.Cu") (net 11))
 (segment (start 146.7235 67.2825) (end 145.4663 66.0253) (width 0.2) (layer "B.Cu") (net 11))
 (segment (start 144.1835 67.2825) (end 145.3158 66.1502) (width 0.2) (layer "F.Cu") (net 33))
 (segment (start 145.3158 66.1502) (end 147.6924 66.1502) (width 0.2) (layer "F.Cu") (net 33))
 (segment (start 147.6924 66.1502) (end 148.0998 65.7428) (width 0.2) (layer "F.Cu") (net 33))
 (segment (start 148.0998 65.1911) (end 148.0998 65.7428) (width 0.2) (layer "F.Cu") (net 33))
 (segment (start 144.7925 67.8912) (end 144.7922 67.8912) (width 0.2) (layer "B.Cu") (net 33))
 (segment (start 144.7925 67.8912) (end 144.184 67.2825) (width 0.2) (layer "B.Cu") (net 33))
 (segment (start 145.401 68.5) (end 144.7925 67.8912) (width 0.2) (layer "B.Cu") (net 33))
 (segment (start 162.324 68.5) (end 145.401 68.5) (width 0.2) (layer "B.Cu") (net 33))
 (segment (start 144.7922 67.8912) (end 144.1835 67.2825) (width 0.2) (layer "B.Cu") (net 33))
 (segment (start 164.27 66.5542) (end 162.324 68.5) (width 0.2) (layer "B.Cu") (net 33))
 (segment (start 157.5643 65.4233) (end 152.4745 65.4233) (width 0.2) (layer "F.Cu") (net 13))
 (segment (start 150.1998 64.3911) (end 150.1998 63.8394) (width 0.2) (layer "F.Cu") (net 13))
 (segment (start 150.8906 63.8394) (end 150.1998 63.8394) (width 0.2) (layer "F.Cu") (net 13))
 (segment (start 159.4235 67.2825) (end 157.5643 65.4233) (width 0.2) (layer "F.Cu") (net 13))
 (segment (start 152.4745 65.4233) (end 150.8906 63.8394) (width 0.2) (layer "F.Cu") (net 13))
 (via (at 152.4745 65.4233) (size 0.6) (drill 0.3) (layers "F.Cu" "B.Cu") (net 13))
 (segment (start 132.7846 71.2717) (end 132.7846 71.9136) (width 0.2) (layer "B.Cu") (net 13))
 (segment (start 137.798 65.4233) (end 136.6589 66.5624) (width 0.2) (layer "B.Cu") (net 13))
 (segment (start 152.4745 65.4233) (end 137.798 65.4233) (width 0.2) (layer "B.Cu") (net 13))
 (segment (start 136.6589 66.5624) (end 133.3759 66.5624) (width 0.2) (layer "B.Cu") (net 13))
 (segment (start 132.6183 67.32) (end 132.6183 71.1054) (width 0.2) (layer "B.Cu") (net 13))
 (segment (start 132.7846 71.9136) (end 132.5 72.1982) (width 0.2) (layer "B.Cu") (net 13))
 (segment (start 132.5 72.1982) (end 132.5 81.8042) (width 0.2) (layer "B.Cu") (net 13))
 (segment (start 132.6183 71.1054) (end 132.7846 71.2717) (width 0.2) (layer "B.Cu") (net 13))
 (segment (start 133.3759 66.5624) (end 132.6183 67.32) (width 0.2) (layer "B.Cu") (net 13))
 (segment (start 132.5 81.8042) (end 131.23 83.0742) (width 0.2) (layer "B.Cu") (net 13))
 (segment (start 129.5 67.0182) (end 129.5 88.9642) (width 0.2) (layer "F.Cu") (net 18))
 (segment (start 129.5 88.9642) (end 131.23 90.6942) (width 0.2) (layer "F.Cu") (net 18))
 (segment (start 150.6532 66.1445) (end 155.7455 66.1445) (width 0.2) (layer "F.Cu") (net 18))
 (segment (start 129.508816 67.009384) (end 129.5 67.0182) (width 0.2) (layer "F.Cu") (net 18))
 (segment (start 149.6998 65.1911) (end 150.6532 66.1445) (width 0.2) (layer "F.Cu") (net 18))
 (segment (start 129.508816 65.365383) (end 129.508816 67.009384) (width 0.2) (layer "F.Cu") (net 18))
 (segment (start 155.7455 66.1445) (end 156.8835 67.2825) (width 0.2) (layer "F.Cu") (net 18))
 (via (at 129.508816 65.365383) (size 0.6) (drill 0.3) (layers "F.Cu" "B.Cu") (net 18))
 (segment (start 153.4271 63.8261) (end 156.8835 67.2825) (width 0.2) (layer "B.Cu") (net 18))
 (segment (start 130.1739 63.8261) (end 153.4271 63.8261) (width 0.2) (layer "B.Cu") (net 18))
 (segment (start 129.508816 65.365383) (end 129.508816 64.491184) (width 0.2) (layer "B.Cu") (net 18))
 (segment (start 129.508816 64.491184) (end 130.1739 63.8261) (width 0.2) (layer "B.Cu") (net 18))
 (segment (start 135.9635 64.1425) (end 132.7257 64.1425) (width 0.2) (layer "F.Cu") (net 15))
 (segment (start 144.1298 65.7428) (end 142.9135 66.9591) (width 0.2) (layer "F.Cu") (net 15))
 (segment (start 139.1035 67.2825) (end 135.9635 64.1425) (width 0.2) (layer "F.Cu") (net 15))
 (segment (start 130.0322 69.9361) (end 130.0322 84.4164) (width 0.2) (layer "F.Cu") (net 15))
 (segment (start 142.1461 68.4287) (end 140.2497 68.4287) (width 0.2) (layer "F.Cu") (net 15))
 (segment (start 147.1998 65.1911) (end 147.1998 65.7428) (width 0.2) (layer "F.Cu") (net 15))
 (segment (start 142.9135 67.6613) (end 142.1461 68.4287) (width 0.2) (layer "F.Cu") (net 15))
 (segment (start 147.1998 65.7428) (end 144.1298 65.7428) (width 0.2) (layer "F.Cu") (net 15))
 (segment (start 132.5 64.3682) (end 132.5 68.2526) (width 0.2) (layer "F.Cu") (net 15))
 (segment (start 140.2497 68.4287) (end 139.1035 67.2825) (width 0.2) (layer "F.Cu") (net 15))
 (segment (start 130.8641 69.1042) (end 130.0322 69.9361) (width 0.2) (layer "F.Cu") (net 15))
 (segment (start 130.0322 84.4164) (end 131.23 85.6142) (width 0.2) (layer "F.Cu") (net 15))
 (segment (start 132.7257 64.1425) (end 132.5 64.3682) (width 0.2) (layer "F.Cu") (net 15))
 (segment (start 132.5 68.2526) (end 131.6484 69.1042) (width 0.2) (layer "F.Cu") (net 15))
 (segment (start 142.9135 66.9591) (end 142.9135 67.6613) (width 0.2) (layer "F.Cu") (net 15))
 (segment (start 131.6484 69.1042) (end 130.8641 69.1042) (width 0.2) (layer "F.Cu") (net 15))
 (segment (start 143.572616 74.427384) (end 145.3519 72.6481) (width 0.2) (layer "F.Cu") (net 12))
 (segment (start 137.190572 74.427384) (end 143.572616 74.427384) (width 0.2) (layer "F.Cu") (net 12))
 (segment (start 147.6151 70.3978) (end 147.6151 69.25) (width 0.2) (layer "F.Cu") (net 12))
 (segment (start 133.77 83.0742) (end 135.969472 80.874728) (width 0.2) (layer "F.Cu") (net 12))
 (segment (start 135.969472 80.874728) (end 135.969472 75.648484) (width 0.2) (layer "F.Cu") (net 12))
 (segment (start 145.3648 72.6481) (end 147.6151 70.3978) (width 0.2) (layer "F.Cu") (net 12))
 (segment (start 145.3519 72.6481) (end 145.3648 72.6481) (width 0.2) (layer "F.Cu") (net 12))
 (segment (start 144.8922 64.3911) (end 147.5998 64.3911) (width 0.2) (layer "F.Cu") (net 12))
 (segment (start 141.6435 67.2825) (end 142.0008 67.2825) (width 0.2) (layer "F.Cu") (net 12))
 (segment (start 142.0008 67.2825) (end 144.8922 64.3911) (width 0.2) (layer "F.Cu") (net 12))
 (segment (start 135.969472 75.648484) (end 137.190572 74.427384) (width 0.2) (layer "F.Cu") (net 12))
 (via (at 147.6151 69.25) (size 0.6) (drill 0.3) (layers "F.Cu" "B.Cu") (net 12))
 (segment (start 141.6435 67.2825) (end 143.611 69.25) (width 0.2) (layer "B.Cu") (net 12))
 (segment (start 143.611 69.25) (end 147.6151 69.25) (width 0.2) (layer "B.Cu") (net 12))
 (segment (start 143.65 70.85) (end 143.65 70) (width 0.2) (layer "B.Cu") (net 3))
 (segment (start 143.65 70) (end 135.936 70) (width 0.2) (layer "B.Cu") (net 3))
 (segment (start 142.5 72.5) (end 142.5 72) (width 0.2) (layer "B.Cu") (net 3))
 (segment (start 142.5 72) (end 143.65 70.85) (width 0.2) (layer "B.Cu") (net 3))
 (segment (start 135.936 70) (end 133.77 67.8342) (width 0.2) (layer "B.Cu") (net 3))
 (segment (start 133.77 70.3742) (end 134.62 71.2242) (width 0.2) (layer "F.Cu") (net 4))
 (segment (start 134.62 71.2242) (end 144.776 71.2242) (width 0.2) (layer "F.Cu") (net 4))
 (segment (start 144.776 71.2242) (end 145 71) (width 0.2) (layer "F.Cu") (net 4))
 (via (at 145 71) (size 0.6) (drill 0.3) (layers "F.Cu" "B.Cu") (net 4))
 (segment (start 145 72) (end 145.8 71.2) (width 0.2) (layer "B.Cu") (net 4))
 (segment (start 145.3 71) (end 145.8 70.5) (width 0.2) (layer "B.Cu") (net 4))
 (segment (start 145 72.5) (end 145 72) (width 0.2) (layer "B.Cu") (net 4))
 (segment (start 145 71) (end 145.3 71) (width 0.2) (layer "B.Cu") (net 4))
 (segment (start 145.8 71.2) (end 145.8 70.5) (width 0.2) (layer "B.Cu") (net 4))
 (segment (start 145.8 70.5) (end 145.8 70) (width 0.2) (layer "B.Cu") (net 4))
 (segment (start 133.77 65.2942) (end 136.5 68.0242) (width 0.2) (layer "F.Cu") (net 1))
 (segment (start 136.5 68.0242) (end 136.5 70.6) (width 0.2) (layer "F.Cu") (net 1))
 (via (at 136.5 70.6) (size 0.6) (drill 0.3) (layers "F.Cu" "B.Cu") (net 1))
 (segment (start 137 72.5) (end 140 72.5) (width 0.2) (layer "B.Cu") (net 1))
 (segment (start 150 69.5) (end 150.248 69.5) (width 0.2) (layer "B.Cu") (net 1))
 (segment (start 136.5 72) (end 137 72.5) (width 0.2) (layer "B.Cu") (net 1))
 (segment (start 149.7225 74.3293) (end 148.9464 73.5532) (width 0.2) (layer "B.Cu") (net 1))
 (segment (start 158.5 70.913901) (end 157.747493 70.161394) (width 0.2) (layer "B.Cu") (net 1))
 (segment (start 158.5 72.5663) (end 157.6042 71.6705) (width 0.2) (layer "B.Cu") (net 1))
 (segment (start 148.9464 73.5532) (end 150 72.5) (width 0.2) (layer "B.Cu") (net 1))
 (segment (start 154.0773 74.3293) (end 149.7225 74.3293) (width 0.2) (layer "B.Cu") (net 1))
 (segment (start 150.651 69.9032) (end 150.651 71.849) (width 0.2) (layer "B.Cu") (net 1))
 (segment (start 154.75 73.6566) (end 154.0773 74.3293) (width 0.2) (layer "B.Cu") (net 1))
 (segment (start 148.746 73.7535) (end 148.9464 73.5532) (width 0.2) (layer "B.Cu") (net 1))
 (segment (start 150.248 69.5) (end 150.651 69.9032) (width 0.2) (layer "B.Cu") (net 1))
 (segment (start 136.5 70.6) (end 136.5 72) (width 0.2) (layer "B.Cu") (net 1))
 (segment (start 154.75 72.3183) (end 154.75 73.6566) (width 0.2) (layer "B.Cu") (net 1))
 (segment (start 158.5 73) (end 158.5 72.5663) (width 0.2) (layer "B.Cu") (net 1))
 (segment (start 141.254 73.7535) (end 148.746 73.7535) (width 0.2) (layer "B.Cu") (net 1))
 (segment (start 158.5 73) (end 158.5 70.913901) (width 0.2) (layer "B.Cu") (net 1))
 (segment (start 150.651 71.849) (end 150 72.5) (width 0.2) (layer "B.Cu") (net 1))
 (segment (start 155.3978 71.6705) (end 154.75 72.3183) (width 0.2) (layer "B.Cu") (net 1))
 (segment (start 140 72.5) (end 141.254 73.7535) (width 0.2) (layer "B.Cu") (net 1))
 (segment (start 157.6042 71.6705) (end 155.3978 71.6705) (width 0.2) (layer "B.Cu") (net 1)))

